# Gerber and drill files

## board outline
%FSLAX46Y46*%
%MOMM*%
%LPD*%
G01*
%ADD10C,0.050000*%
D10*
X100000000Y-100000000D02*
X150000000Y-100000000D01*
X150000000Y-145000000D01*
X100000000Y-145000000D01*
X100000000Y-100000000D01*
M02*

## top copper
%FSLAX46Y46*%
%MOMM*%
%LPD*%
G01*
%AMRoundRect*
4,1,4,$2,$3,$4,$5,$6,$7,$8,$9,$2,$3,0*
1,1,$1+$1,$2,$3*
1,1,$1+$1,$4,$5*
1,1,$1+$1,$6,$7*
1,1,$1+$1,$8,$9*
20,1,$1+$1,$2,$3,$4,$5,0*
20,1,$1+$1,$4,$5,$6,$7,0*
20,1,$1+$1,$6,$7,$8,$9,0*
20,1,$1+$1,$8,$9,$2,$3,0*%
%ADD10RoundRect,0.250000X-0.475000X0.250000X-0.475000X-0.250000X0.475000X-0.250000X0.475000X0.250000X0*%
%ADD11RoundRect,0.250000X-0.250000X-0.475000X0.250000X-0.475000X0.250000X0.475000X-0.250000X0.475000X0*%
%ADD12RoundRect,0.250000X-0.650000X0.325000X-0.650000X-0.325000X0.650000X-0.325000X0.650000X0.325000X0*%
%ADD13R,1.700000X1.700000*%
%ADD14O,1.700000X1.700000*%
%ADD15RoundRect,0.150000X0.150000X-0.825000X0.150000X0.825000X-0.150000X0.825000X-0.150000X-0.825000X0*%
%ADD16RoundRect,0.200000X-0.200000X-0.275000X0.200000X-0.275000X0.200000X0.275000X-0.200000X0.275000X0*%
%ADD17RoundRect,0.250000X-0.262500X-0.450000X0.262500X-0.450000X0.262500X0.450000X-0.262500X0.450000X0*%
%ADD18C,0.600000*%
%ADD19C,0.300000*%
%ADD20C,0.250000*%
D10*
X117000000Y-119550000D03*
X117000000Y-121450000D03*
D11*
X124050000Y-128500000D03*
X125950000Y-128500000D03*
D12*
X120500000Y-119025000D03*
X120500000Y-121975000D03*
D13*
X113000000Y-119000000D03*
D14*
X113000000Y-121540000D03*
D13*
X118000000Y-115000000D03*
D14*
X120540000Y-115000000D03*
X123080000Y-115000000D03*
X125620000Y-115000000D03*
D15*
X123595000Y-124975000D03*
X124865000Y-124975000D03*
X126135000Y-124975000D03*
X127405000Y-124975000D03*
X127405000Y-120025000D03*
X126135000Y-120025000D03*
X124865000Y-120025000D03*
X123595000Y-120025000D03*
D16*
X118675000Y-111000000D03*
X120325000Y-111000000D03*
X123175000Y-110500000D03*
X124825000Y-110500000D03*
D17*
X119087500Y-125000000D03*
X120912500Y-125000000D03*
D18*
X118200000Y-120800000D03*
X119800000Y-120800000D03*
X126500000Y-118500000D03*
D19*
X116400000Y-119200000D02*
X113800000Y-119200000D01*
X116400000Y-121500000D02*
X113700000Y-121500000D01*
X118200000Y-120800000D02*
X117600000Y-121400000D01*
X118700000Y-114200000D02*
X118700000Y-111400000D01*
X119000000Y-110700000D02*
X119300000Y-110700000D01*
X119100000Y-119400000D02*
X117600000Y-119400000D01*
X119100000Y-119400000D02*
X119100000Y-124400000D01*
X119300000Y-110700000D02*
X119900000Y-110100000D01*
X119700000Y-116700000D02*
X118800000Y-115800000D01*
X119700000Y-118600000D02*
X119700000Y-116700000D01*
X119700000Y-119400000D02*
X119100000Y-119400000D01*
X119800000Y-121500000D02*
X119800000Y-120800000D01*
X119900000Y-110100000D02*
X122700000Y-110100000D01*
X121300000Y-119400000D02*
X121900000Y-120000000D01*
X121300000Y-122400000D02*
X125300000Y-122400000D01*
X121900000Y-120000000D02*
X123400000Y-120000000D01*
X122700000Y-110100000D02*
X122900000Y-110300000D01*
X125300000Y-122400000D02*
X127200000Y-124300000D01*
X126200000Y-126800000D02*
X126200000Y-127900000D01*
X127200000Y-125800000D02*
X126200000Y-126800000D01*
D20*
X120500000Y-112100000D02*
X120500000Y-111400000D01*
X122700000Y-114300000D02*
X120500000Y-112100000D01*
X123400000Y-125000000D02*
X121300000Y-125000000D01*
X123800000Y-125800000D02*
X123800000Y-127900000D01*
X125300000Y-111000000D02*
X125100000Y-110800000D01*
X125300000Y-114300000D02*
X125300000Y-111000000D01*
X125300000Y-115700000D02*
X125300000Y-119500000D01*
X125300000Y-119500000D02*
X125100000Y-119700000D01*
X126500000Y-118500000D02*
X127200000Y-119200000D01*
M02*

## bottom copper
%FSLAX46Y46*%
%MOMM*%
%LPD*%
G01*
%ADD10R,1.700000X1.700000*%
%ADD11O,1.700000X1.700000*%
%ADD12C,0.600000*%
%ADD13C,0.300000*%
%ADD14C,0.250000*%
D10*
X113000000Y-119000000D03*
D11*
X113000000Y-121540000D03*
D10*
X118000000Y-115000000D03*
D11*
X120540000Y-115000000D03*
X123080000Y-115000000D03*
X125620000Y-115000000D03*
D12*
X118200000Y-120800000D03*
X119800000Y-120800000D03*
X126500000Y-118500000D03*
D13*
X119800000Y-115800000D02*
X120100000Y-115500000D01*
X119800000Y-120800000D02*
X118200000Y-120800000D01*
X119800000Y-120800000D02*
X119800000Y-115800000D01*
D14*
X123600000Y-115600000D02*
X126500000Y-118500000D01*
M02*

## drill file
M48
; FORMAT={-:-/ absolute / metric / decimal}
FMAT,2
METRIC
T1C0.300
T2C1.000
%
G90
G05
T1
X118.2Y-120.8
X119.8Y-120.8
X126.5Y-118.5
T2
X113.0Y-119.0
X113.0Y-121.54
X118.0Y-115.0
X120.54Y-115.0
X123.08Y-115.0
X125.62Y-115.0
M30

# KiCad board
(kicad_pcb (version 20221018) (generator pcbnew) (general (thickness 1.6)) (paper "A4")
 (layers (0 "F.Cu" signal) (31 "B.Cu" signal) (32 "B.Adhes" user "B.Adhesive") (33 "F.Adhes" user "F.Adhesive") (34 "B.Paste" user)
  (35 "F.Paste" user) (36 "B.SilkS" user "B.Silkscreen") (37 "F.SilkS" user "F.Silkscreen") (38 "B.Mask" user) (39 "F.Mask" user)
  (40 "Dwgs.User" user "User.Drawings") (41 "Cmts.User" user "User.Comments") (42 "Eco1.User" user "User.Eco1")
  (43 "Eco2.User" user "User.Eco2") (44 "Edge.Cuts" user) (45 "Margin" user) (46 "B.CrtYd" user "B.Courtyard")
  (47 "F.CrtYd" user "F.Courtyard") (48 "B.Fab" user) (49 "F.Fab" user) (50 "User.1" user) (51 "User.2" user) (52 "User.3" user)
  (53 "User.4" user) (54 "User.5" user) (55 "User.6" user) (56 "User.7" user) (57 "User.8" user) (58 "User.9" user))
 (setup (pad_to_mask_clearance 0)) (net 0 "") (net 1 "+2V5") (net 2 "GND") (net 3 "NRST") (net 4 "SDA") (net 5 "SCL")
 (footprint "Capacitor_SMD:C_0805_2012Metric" (layer "F.Cu") (at 117 120.5 -90)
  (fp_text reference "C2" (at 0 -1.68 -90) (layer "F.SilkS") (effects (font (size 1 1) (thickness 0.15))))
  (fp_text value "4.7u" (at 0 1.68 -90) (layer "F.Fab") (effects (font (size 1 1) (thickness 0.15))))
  (pad "1" smd roundrect (at -0.95 0 270) (size 1 1.45) (layers "F.Cu" "F.Paste" "F.Mask") (roundrect_rratio 0.25) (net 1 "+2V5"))
  (pad "2" smd roundrect (at 0.95 0 270) (size 1 1.45) (layers "F.Cu" "F.Paste" "F.Mask") (roundrect_rratio 0.25) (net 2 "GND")))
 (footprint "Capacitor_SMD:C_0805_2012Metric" (layer "F.Cu") (at 125 128.5)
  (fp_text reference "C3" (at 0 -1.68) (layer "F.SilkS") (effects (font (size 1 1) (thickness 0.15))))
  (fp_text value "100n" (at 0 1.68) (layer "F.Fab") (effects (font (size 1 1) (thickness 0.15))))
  (pad "1" smd roundrect (at -0.95 0) (size 1 1.45) (layers "F.Cu" "F.Paste" "F.Mask") (roundrect_rratio 0.25) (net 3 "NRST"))
  (pad "2" smd roundrect (at 0.95 0) (size 1 1.45) (layers "F.Cu" "F.Paste" "F.Mask") (roundrect_rratio 0.25) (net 2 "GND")))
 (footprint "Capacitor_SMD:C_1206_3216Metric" (layer "F.Cu") (at 120.5 120.5 -90)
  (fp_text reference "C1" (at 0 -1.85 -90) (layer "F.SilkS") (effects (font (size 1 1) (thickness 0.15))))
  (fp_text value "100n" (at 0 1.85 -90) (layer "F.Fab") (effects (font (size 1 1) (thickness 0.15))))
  (pad "1" smd roundrect (at -1.475 0 270) (size 1.15 1.8) (layers "F.Cu" "F.Paste" "F.Mask") (roundrect_rratio 0.217391) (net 1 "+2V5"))
  (pad "2" smd roundrect (at 1.475 0 270) (size 1.15 1.8) (layers "F.Cu" "F.Paste" "F.Mask") (roundrect_rratio 0.217391) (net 2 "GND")))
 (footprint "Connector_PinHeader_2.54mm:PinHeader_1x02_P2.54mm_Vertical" (layer "F.Cu") (at 113 119)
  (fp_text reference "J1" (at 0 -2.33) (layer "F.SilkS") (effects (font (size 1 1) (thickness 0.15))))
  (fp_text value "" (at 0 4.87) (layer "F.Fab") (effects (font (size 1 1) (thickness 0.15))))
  (pad "1" thru_hole rect (at 0 0) (size 1.7 1.7) (drill 1) (layers "*.Cu" "*.Mask") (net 1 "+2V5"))
  (pad "2" thru_hole oval (at 0 2.54) (size 1.7 1.7) (drill 1) (layers "*.Cu" "*.Mask") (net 2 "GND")))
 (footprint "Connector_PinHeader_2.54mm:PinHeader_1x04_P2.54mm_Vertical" (layer "F.Cu") (at 118 115 90)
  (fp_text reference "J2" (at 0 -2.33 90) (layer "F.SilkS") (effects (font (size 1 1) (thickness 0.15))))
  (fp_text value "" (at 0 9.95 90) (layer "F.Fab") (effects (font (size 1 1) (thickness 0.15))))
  (pad "1" thru_hole rect (at 0 0 90) (size 1.7 1.7) (drill 1) (layers "*.Cu" "*.Mask") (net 1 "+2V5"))
  (pad "2" thru_hole oval (at 0 2.54 90) (size 1.7 1.7) (drill 1) (layers "*.Cu" "*.Mask") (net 2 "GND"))
  (pad "3" thru_hole oval (at 0 5.08 90) (size 1.7 1.7) (drill 1) (layers "*.Cu" "*.Mask") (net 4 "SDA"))
  (pad "4" thru_hole oval (at 0 7.62 90) (size 1.7 1.7) (drill 1) (layers "*.Cu" "*.Mask") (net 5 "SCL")))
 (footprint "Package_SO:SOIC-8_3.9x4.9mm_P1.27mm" (layer "F.Cu") (at 125.5 122.5 90)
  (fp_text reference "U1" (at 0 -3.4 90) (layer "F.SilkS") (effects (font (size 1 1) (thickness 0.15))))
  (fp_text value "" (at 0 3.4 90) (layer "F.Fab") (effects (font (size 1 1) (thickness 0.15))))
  (pad "1" smd roundrect (at -2.475 -1.905 90) (size 1.95 0.6) (layers "F.Cu" "F.Paste" "F.Mask") (roundrect_rratio 0.25) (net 3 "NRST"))
  (pad "2" smd roundrect (at -2.475 -0.635 90) (size 1.95 0.6) (layers "F.Cu" "F.Paste" "F.Mask") (roundrect_rratio 0.25))
  (pad "3" smd roundrect (at -2.475 0.635 90) (size 1.95 0.6) (layers "F.Cu" "F.Paste" "F.Mask") (roundrect_rratio 0.25))
  (pad "4" smd roundrect (at -2.475 1.905 90) (size 1.95 0.6) (layers "F.Cu" "F.Paste" "F.Mask") (roundrect_rratio 0.25) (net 2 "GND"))
  (pad "5" smd roundrect (at 2.475 1.905 90) (size 1.95 0.6) (layers "F.Cu" "F.Paste" "F.Mask") (roundrect_rratio 0.25) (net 4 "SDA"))
  (pad "6" smd roundrect (at 2.475 0.635 90) (size 1.95 0.6) (layers "F.Cu" "F.Paste" "F.Mask") (roundrect_rratio 0.25))
  (pad "7" smd roundrect (at 2.475 -0.635 90) (size 1.95 0.6) (layers "F.Cu" "F.Paste" "F.Mask") (roundrect_rratio 0.25) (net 5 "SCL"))
  (pad "8" smd roundrect (at 2.475 -1.905 90) (size 1.95 0.6) (layers "F.Cu" "F.Paste" "F.Mask") (roundrect_rratio 0.25) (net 1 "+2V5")))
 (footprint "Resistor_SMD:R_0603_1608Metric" (layer "F.Cu") (at 119.5 111)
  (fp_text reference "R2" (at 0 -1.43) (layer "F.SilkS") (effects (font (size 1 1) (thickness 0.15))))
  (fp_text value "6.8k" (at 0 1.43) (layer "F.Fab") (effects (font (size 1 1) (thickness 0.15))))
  (pad "1" smd roundrect (at -0.825 0) (size 0.8 0.95) (layers "F.Cu" "F.Paste" "F.Mask") (roundrect_rratio 0.25) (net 1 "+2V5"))
  (pad "2" smd roundrect (at 0.825 0) (size 0.8 0.95) (layers "F.Cu" "F.Paste" "F.Mask") (roundrect_rratio 0.25) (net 4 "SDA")))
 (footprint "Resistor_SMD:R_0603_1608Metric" (layer "F.Cu") (at 124 110.5)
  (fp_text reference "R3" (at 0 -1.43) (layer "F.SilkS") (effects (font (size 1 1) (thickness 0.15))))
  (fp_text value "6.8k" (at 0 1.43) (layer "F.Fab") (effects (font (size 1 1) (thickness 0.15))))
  (pad "1" smd roundrect (at -0.825 0) (size 0.8 0.95) (layers "F.Cu" "F.Paste" "F.Mask") (roundrect_rratio 0.25) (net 1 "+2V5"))
  (pad "2" smd roundrect (at 0.825 0) (size 0.8 0.95) (layers "F.Cu" "F.Paste" "F.Mask") (roundrect_rratio 0.25) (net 5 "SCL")))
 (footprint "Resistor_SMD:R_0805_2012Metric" (layer "F.Cu") (at 120 125)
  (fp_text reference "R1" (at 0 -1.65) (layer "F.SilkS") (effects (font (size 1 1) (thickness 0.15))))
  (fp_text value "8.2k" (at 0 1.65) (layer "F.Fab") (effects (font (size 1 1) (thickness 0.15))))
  (pad "1" smd roundrect (at -0.9125 0) (size 1.025 1.4) (layers "F.Cu" "F.Paste" "F.Mask") (roundrect_rratio 0.243902) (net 1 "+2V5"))
  (pad "2" smd roundrect (at 0.9125 0) (size 1.025 1.4) (layers "F.Cu" "F.Paste" "F.Mask") (roundrect_rratio 0.243902) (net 3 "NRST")))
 (gr_rect (start 100 100) (end 150 145) (stroke (width 0.05) (type default)) (fill none) (layer "Edge.Cuts"))
 (segment (start 116.4 119.2) (end 113.8 119.2) (width 0.3) (layer "F.Cu") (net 1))
 (segment (start 116.4 121.5) (end 113.7 121.5) (width 0.3) (layer "F.Cu") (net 2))
 (segment (start 118.2 120.8) (end 117.6 121.4) (width 0.3) (layer "F.Cu") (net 2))
 (segment (start 118.7 114.2) (end 118.7 111.4) (width 0.3) (layer "F.Cu") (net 1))
 (segment (start 119 110.7) (end 119.3 110.7) (width 0.3) (layer "F.Cu") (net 1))
 (segment (start 119.1 119.4) (end 117.6 119.4) (width 0.3) (layer "F.Cu") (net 1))
 (segment (start 119.1 119.4) (end 119.1 124.4) (width 0.3) (layer "F.Cu") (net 1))
 (segment (start 119.3 110.7) (end 119.9 110.1) (width 0.3) (layer "F.Cu") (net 1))
 (segment (start 119.7 116.7) (end 118.8 115.8) (width 0.3) (layer "F.Cu") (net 1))
 (segment (start 119.7 118.6) (end 119.7 116.7) (width 0.3) (layer "F.Cu") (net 1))
 (segment (start 119.7 119.4) (end 119.1 119.4) (width 0.3) (layer "F.Cu") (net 1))
 (segment (start 119.8 121.5) (end 119.8 120.8) (width 0.3) (layer "F.Cu") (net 2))
 (segment (start 119.9 110.1) (end 122.7 110.1) (width 0.3) (layer "F.Cu") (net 1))
 (segment (start 121.3 119.4) (end 121.9 120) (width 0.3) (layer "F.Cu") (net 1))
 (segment (start 121.3 122.4) (end 125.3 122.4) (width 0.3) (layer "F.Cu") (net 2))
 (segment (start 121.9 120) (end 123.4 120) (width 0.3) (layer "F.Cu") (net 1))
 (segment (start 122.7 110.1) (end 122.9 110.3) (width 0.3) (layer "F.Cu") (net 1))
 (segment (start 125.3 122.4) (end 127.2 124.3) (width 0.3) (layer "F.Cu") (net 2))
 (segment (start 126.2 126.8) (end 126.2 127.9) (width 0.3) (layer "F.Cu") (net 2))
 (segment (start 127.2 125.8) (end 126.2 126.8) (width 0.3) (layer "F.Cu") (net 2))
 (via (at 118.2 120.8) (size 0.6) (drill 0.3) (layers "F.Cu" "B.Cu") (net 2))
 (via (at 119.8 120.8) (size 0.6) (drill 0.3) (layers "F.Cu" "B.Cu") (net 2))
 (segment (start 119.8 115.8) (end 120.1 115.5) (width 0.3) (layer "B.Cu") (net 2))
 (segment (start 119.8 120.8) (end 118.2 120.8) (width 0.3) (layer "B.Cu") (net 2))
 (segment (start 119.8 120.8) (end 119.8 115.8) (width 0.3) (layer "B.Cu") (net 2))
 (segment (start 120.5 112.1) (end 120.5 111.4) (width 0.25) (layer "F.Cu") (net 4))
 (segment (start 122.7 114.3) (end 120.5 112.1) (width 0.25) (layer "F.Cu") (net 4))
 (segment (start 123.4 125) (end 121.3 125) (width 0.25) (layer "F.Cu") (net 3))
 (segment (start 123.8 125.8) (end 123.8 127.9) (width 0.25) (layer "F.Cu") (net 3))
 (segment (start 125.3 111) (end 125.1 110.8) (width 0.25) (layer "F.Cu") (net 5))
 (segment (start 125.3 114.3) (end 125.3 111) (width 0.25) (layer "F.Cu") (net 5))
 (segment (start 125.3 115.7) (end 125.3 119.5) (width 0.25) (layer "F.Cu") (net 5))
 (segment (start 125.3 119.5) (end 125.1 119.7) (width 0.25) (layer "F.Cu") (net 5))
 (segment (start 126.5 118.5) (end 127.2 119.2) (width 0.25) (layer "F.Cu") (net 4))
 (via (at 126.5 118.5) (size 0.6) (drill 0.3) (layers "F.Cu" "B.Cu") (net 4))
 (segment (start 123.6 115.6) (end 126.5 118.5) (width 0.25) (layer "B.Cu") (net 4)))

